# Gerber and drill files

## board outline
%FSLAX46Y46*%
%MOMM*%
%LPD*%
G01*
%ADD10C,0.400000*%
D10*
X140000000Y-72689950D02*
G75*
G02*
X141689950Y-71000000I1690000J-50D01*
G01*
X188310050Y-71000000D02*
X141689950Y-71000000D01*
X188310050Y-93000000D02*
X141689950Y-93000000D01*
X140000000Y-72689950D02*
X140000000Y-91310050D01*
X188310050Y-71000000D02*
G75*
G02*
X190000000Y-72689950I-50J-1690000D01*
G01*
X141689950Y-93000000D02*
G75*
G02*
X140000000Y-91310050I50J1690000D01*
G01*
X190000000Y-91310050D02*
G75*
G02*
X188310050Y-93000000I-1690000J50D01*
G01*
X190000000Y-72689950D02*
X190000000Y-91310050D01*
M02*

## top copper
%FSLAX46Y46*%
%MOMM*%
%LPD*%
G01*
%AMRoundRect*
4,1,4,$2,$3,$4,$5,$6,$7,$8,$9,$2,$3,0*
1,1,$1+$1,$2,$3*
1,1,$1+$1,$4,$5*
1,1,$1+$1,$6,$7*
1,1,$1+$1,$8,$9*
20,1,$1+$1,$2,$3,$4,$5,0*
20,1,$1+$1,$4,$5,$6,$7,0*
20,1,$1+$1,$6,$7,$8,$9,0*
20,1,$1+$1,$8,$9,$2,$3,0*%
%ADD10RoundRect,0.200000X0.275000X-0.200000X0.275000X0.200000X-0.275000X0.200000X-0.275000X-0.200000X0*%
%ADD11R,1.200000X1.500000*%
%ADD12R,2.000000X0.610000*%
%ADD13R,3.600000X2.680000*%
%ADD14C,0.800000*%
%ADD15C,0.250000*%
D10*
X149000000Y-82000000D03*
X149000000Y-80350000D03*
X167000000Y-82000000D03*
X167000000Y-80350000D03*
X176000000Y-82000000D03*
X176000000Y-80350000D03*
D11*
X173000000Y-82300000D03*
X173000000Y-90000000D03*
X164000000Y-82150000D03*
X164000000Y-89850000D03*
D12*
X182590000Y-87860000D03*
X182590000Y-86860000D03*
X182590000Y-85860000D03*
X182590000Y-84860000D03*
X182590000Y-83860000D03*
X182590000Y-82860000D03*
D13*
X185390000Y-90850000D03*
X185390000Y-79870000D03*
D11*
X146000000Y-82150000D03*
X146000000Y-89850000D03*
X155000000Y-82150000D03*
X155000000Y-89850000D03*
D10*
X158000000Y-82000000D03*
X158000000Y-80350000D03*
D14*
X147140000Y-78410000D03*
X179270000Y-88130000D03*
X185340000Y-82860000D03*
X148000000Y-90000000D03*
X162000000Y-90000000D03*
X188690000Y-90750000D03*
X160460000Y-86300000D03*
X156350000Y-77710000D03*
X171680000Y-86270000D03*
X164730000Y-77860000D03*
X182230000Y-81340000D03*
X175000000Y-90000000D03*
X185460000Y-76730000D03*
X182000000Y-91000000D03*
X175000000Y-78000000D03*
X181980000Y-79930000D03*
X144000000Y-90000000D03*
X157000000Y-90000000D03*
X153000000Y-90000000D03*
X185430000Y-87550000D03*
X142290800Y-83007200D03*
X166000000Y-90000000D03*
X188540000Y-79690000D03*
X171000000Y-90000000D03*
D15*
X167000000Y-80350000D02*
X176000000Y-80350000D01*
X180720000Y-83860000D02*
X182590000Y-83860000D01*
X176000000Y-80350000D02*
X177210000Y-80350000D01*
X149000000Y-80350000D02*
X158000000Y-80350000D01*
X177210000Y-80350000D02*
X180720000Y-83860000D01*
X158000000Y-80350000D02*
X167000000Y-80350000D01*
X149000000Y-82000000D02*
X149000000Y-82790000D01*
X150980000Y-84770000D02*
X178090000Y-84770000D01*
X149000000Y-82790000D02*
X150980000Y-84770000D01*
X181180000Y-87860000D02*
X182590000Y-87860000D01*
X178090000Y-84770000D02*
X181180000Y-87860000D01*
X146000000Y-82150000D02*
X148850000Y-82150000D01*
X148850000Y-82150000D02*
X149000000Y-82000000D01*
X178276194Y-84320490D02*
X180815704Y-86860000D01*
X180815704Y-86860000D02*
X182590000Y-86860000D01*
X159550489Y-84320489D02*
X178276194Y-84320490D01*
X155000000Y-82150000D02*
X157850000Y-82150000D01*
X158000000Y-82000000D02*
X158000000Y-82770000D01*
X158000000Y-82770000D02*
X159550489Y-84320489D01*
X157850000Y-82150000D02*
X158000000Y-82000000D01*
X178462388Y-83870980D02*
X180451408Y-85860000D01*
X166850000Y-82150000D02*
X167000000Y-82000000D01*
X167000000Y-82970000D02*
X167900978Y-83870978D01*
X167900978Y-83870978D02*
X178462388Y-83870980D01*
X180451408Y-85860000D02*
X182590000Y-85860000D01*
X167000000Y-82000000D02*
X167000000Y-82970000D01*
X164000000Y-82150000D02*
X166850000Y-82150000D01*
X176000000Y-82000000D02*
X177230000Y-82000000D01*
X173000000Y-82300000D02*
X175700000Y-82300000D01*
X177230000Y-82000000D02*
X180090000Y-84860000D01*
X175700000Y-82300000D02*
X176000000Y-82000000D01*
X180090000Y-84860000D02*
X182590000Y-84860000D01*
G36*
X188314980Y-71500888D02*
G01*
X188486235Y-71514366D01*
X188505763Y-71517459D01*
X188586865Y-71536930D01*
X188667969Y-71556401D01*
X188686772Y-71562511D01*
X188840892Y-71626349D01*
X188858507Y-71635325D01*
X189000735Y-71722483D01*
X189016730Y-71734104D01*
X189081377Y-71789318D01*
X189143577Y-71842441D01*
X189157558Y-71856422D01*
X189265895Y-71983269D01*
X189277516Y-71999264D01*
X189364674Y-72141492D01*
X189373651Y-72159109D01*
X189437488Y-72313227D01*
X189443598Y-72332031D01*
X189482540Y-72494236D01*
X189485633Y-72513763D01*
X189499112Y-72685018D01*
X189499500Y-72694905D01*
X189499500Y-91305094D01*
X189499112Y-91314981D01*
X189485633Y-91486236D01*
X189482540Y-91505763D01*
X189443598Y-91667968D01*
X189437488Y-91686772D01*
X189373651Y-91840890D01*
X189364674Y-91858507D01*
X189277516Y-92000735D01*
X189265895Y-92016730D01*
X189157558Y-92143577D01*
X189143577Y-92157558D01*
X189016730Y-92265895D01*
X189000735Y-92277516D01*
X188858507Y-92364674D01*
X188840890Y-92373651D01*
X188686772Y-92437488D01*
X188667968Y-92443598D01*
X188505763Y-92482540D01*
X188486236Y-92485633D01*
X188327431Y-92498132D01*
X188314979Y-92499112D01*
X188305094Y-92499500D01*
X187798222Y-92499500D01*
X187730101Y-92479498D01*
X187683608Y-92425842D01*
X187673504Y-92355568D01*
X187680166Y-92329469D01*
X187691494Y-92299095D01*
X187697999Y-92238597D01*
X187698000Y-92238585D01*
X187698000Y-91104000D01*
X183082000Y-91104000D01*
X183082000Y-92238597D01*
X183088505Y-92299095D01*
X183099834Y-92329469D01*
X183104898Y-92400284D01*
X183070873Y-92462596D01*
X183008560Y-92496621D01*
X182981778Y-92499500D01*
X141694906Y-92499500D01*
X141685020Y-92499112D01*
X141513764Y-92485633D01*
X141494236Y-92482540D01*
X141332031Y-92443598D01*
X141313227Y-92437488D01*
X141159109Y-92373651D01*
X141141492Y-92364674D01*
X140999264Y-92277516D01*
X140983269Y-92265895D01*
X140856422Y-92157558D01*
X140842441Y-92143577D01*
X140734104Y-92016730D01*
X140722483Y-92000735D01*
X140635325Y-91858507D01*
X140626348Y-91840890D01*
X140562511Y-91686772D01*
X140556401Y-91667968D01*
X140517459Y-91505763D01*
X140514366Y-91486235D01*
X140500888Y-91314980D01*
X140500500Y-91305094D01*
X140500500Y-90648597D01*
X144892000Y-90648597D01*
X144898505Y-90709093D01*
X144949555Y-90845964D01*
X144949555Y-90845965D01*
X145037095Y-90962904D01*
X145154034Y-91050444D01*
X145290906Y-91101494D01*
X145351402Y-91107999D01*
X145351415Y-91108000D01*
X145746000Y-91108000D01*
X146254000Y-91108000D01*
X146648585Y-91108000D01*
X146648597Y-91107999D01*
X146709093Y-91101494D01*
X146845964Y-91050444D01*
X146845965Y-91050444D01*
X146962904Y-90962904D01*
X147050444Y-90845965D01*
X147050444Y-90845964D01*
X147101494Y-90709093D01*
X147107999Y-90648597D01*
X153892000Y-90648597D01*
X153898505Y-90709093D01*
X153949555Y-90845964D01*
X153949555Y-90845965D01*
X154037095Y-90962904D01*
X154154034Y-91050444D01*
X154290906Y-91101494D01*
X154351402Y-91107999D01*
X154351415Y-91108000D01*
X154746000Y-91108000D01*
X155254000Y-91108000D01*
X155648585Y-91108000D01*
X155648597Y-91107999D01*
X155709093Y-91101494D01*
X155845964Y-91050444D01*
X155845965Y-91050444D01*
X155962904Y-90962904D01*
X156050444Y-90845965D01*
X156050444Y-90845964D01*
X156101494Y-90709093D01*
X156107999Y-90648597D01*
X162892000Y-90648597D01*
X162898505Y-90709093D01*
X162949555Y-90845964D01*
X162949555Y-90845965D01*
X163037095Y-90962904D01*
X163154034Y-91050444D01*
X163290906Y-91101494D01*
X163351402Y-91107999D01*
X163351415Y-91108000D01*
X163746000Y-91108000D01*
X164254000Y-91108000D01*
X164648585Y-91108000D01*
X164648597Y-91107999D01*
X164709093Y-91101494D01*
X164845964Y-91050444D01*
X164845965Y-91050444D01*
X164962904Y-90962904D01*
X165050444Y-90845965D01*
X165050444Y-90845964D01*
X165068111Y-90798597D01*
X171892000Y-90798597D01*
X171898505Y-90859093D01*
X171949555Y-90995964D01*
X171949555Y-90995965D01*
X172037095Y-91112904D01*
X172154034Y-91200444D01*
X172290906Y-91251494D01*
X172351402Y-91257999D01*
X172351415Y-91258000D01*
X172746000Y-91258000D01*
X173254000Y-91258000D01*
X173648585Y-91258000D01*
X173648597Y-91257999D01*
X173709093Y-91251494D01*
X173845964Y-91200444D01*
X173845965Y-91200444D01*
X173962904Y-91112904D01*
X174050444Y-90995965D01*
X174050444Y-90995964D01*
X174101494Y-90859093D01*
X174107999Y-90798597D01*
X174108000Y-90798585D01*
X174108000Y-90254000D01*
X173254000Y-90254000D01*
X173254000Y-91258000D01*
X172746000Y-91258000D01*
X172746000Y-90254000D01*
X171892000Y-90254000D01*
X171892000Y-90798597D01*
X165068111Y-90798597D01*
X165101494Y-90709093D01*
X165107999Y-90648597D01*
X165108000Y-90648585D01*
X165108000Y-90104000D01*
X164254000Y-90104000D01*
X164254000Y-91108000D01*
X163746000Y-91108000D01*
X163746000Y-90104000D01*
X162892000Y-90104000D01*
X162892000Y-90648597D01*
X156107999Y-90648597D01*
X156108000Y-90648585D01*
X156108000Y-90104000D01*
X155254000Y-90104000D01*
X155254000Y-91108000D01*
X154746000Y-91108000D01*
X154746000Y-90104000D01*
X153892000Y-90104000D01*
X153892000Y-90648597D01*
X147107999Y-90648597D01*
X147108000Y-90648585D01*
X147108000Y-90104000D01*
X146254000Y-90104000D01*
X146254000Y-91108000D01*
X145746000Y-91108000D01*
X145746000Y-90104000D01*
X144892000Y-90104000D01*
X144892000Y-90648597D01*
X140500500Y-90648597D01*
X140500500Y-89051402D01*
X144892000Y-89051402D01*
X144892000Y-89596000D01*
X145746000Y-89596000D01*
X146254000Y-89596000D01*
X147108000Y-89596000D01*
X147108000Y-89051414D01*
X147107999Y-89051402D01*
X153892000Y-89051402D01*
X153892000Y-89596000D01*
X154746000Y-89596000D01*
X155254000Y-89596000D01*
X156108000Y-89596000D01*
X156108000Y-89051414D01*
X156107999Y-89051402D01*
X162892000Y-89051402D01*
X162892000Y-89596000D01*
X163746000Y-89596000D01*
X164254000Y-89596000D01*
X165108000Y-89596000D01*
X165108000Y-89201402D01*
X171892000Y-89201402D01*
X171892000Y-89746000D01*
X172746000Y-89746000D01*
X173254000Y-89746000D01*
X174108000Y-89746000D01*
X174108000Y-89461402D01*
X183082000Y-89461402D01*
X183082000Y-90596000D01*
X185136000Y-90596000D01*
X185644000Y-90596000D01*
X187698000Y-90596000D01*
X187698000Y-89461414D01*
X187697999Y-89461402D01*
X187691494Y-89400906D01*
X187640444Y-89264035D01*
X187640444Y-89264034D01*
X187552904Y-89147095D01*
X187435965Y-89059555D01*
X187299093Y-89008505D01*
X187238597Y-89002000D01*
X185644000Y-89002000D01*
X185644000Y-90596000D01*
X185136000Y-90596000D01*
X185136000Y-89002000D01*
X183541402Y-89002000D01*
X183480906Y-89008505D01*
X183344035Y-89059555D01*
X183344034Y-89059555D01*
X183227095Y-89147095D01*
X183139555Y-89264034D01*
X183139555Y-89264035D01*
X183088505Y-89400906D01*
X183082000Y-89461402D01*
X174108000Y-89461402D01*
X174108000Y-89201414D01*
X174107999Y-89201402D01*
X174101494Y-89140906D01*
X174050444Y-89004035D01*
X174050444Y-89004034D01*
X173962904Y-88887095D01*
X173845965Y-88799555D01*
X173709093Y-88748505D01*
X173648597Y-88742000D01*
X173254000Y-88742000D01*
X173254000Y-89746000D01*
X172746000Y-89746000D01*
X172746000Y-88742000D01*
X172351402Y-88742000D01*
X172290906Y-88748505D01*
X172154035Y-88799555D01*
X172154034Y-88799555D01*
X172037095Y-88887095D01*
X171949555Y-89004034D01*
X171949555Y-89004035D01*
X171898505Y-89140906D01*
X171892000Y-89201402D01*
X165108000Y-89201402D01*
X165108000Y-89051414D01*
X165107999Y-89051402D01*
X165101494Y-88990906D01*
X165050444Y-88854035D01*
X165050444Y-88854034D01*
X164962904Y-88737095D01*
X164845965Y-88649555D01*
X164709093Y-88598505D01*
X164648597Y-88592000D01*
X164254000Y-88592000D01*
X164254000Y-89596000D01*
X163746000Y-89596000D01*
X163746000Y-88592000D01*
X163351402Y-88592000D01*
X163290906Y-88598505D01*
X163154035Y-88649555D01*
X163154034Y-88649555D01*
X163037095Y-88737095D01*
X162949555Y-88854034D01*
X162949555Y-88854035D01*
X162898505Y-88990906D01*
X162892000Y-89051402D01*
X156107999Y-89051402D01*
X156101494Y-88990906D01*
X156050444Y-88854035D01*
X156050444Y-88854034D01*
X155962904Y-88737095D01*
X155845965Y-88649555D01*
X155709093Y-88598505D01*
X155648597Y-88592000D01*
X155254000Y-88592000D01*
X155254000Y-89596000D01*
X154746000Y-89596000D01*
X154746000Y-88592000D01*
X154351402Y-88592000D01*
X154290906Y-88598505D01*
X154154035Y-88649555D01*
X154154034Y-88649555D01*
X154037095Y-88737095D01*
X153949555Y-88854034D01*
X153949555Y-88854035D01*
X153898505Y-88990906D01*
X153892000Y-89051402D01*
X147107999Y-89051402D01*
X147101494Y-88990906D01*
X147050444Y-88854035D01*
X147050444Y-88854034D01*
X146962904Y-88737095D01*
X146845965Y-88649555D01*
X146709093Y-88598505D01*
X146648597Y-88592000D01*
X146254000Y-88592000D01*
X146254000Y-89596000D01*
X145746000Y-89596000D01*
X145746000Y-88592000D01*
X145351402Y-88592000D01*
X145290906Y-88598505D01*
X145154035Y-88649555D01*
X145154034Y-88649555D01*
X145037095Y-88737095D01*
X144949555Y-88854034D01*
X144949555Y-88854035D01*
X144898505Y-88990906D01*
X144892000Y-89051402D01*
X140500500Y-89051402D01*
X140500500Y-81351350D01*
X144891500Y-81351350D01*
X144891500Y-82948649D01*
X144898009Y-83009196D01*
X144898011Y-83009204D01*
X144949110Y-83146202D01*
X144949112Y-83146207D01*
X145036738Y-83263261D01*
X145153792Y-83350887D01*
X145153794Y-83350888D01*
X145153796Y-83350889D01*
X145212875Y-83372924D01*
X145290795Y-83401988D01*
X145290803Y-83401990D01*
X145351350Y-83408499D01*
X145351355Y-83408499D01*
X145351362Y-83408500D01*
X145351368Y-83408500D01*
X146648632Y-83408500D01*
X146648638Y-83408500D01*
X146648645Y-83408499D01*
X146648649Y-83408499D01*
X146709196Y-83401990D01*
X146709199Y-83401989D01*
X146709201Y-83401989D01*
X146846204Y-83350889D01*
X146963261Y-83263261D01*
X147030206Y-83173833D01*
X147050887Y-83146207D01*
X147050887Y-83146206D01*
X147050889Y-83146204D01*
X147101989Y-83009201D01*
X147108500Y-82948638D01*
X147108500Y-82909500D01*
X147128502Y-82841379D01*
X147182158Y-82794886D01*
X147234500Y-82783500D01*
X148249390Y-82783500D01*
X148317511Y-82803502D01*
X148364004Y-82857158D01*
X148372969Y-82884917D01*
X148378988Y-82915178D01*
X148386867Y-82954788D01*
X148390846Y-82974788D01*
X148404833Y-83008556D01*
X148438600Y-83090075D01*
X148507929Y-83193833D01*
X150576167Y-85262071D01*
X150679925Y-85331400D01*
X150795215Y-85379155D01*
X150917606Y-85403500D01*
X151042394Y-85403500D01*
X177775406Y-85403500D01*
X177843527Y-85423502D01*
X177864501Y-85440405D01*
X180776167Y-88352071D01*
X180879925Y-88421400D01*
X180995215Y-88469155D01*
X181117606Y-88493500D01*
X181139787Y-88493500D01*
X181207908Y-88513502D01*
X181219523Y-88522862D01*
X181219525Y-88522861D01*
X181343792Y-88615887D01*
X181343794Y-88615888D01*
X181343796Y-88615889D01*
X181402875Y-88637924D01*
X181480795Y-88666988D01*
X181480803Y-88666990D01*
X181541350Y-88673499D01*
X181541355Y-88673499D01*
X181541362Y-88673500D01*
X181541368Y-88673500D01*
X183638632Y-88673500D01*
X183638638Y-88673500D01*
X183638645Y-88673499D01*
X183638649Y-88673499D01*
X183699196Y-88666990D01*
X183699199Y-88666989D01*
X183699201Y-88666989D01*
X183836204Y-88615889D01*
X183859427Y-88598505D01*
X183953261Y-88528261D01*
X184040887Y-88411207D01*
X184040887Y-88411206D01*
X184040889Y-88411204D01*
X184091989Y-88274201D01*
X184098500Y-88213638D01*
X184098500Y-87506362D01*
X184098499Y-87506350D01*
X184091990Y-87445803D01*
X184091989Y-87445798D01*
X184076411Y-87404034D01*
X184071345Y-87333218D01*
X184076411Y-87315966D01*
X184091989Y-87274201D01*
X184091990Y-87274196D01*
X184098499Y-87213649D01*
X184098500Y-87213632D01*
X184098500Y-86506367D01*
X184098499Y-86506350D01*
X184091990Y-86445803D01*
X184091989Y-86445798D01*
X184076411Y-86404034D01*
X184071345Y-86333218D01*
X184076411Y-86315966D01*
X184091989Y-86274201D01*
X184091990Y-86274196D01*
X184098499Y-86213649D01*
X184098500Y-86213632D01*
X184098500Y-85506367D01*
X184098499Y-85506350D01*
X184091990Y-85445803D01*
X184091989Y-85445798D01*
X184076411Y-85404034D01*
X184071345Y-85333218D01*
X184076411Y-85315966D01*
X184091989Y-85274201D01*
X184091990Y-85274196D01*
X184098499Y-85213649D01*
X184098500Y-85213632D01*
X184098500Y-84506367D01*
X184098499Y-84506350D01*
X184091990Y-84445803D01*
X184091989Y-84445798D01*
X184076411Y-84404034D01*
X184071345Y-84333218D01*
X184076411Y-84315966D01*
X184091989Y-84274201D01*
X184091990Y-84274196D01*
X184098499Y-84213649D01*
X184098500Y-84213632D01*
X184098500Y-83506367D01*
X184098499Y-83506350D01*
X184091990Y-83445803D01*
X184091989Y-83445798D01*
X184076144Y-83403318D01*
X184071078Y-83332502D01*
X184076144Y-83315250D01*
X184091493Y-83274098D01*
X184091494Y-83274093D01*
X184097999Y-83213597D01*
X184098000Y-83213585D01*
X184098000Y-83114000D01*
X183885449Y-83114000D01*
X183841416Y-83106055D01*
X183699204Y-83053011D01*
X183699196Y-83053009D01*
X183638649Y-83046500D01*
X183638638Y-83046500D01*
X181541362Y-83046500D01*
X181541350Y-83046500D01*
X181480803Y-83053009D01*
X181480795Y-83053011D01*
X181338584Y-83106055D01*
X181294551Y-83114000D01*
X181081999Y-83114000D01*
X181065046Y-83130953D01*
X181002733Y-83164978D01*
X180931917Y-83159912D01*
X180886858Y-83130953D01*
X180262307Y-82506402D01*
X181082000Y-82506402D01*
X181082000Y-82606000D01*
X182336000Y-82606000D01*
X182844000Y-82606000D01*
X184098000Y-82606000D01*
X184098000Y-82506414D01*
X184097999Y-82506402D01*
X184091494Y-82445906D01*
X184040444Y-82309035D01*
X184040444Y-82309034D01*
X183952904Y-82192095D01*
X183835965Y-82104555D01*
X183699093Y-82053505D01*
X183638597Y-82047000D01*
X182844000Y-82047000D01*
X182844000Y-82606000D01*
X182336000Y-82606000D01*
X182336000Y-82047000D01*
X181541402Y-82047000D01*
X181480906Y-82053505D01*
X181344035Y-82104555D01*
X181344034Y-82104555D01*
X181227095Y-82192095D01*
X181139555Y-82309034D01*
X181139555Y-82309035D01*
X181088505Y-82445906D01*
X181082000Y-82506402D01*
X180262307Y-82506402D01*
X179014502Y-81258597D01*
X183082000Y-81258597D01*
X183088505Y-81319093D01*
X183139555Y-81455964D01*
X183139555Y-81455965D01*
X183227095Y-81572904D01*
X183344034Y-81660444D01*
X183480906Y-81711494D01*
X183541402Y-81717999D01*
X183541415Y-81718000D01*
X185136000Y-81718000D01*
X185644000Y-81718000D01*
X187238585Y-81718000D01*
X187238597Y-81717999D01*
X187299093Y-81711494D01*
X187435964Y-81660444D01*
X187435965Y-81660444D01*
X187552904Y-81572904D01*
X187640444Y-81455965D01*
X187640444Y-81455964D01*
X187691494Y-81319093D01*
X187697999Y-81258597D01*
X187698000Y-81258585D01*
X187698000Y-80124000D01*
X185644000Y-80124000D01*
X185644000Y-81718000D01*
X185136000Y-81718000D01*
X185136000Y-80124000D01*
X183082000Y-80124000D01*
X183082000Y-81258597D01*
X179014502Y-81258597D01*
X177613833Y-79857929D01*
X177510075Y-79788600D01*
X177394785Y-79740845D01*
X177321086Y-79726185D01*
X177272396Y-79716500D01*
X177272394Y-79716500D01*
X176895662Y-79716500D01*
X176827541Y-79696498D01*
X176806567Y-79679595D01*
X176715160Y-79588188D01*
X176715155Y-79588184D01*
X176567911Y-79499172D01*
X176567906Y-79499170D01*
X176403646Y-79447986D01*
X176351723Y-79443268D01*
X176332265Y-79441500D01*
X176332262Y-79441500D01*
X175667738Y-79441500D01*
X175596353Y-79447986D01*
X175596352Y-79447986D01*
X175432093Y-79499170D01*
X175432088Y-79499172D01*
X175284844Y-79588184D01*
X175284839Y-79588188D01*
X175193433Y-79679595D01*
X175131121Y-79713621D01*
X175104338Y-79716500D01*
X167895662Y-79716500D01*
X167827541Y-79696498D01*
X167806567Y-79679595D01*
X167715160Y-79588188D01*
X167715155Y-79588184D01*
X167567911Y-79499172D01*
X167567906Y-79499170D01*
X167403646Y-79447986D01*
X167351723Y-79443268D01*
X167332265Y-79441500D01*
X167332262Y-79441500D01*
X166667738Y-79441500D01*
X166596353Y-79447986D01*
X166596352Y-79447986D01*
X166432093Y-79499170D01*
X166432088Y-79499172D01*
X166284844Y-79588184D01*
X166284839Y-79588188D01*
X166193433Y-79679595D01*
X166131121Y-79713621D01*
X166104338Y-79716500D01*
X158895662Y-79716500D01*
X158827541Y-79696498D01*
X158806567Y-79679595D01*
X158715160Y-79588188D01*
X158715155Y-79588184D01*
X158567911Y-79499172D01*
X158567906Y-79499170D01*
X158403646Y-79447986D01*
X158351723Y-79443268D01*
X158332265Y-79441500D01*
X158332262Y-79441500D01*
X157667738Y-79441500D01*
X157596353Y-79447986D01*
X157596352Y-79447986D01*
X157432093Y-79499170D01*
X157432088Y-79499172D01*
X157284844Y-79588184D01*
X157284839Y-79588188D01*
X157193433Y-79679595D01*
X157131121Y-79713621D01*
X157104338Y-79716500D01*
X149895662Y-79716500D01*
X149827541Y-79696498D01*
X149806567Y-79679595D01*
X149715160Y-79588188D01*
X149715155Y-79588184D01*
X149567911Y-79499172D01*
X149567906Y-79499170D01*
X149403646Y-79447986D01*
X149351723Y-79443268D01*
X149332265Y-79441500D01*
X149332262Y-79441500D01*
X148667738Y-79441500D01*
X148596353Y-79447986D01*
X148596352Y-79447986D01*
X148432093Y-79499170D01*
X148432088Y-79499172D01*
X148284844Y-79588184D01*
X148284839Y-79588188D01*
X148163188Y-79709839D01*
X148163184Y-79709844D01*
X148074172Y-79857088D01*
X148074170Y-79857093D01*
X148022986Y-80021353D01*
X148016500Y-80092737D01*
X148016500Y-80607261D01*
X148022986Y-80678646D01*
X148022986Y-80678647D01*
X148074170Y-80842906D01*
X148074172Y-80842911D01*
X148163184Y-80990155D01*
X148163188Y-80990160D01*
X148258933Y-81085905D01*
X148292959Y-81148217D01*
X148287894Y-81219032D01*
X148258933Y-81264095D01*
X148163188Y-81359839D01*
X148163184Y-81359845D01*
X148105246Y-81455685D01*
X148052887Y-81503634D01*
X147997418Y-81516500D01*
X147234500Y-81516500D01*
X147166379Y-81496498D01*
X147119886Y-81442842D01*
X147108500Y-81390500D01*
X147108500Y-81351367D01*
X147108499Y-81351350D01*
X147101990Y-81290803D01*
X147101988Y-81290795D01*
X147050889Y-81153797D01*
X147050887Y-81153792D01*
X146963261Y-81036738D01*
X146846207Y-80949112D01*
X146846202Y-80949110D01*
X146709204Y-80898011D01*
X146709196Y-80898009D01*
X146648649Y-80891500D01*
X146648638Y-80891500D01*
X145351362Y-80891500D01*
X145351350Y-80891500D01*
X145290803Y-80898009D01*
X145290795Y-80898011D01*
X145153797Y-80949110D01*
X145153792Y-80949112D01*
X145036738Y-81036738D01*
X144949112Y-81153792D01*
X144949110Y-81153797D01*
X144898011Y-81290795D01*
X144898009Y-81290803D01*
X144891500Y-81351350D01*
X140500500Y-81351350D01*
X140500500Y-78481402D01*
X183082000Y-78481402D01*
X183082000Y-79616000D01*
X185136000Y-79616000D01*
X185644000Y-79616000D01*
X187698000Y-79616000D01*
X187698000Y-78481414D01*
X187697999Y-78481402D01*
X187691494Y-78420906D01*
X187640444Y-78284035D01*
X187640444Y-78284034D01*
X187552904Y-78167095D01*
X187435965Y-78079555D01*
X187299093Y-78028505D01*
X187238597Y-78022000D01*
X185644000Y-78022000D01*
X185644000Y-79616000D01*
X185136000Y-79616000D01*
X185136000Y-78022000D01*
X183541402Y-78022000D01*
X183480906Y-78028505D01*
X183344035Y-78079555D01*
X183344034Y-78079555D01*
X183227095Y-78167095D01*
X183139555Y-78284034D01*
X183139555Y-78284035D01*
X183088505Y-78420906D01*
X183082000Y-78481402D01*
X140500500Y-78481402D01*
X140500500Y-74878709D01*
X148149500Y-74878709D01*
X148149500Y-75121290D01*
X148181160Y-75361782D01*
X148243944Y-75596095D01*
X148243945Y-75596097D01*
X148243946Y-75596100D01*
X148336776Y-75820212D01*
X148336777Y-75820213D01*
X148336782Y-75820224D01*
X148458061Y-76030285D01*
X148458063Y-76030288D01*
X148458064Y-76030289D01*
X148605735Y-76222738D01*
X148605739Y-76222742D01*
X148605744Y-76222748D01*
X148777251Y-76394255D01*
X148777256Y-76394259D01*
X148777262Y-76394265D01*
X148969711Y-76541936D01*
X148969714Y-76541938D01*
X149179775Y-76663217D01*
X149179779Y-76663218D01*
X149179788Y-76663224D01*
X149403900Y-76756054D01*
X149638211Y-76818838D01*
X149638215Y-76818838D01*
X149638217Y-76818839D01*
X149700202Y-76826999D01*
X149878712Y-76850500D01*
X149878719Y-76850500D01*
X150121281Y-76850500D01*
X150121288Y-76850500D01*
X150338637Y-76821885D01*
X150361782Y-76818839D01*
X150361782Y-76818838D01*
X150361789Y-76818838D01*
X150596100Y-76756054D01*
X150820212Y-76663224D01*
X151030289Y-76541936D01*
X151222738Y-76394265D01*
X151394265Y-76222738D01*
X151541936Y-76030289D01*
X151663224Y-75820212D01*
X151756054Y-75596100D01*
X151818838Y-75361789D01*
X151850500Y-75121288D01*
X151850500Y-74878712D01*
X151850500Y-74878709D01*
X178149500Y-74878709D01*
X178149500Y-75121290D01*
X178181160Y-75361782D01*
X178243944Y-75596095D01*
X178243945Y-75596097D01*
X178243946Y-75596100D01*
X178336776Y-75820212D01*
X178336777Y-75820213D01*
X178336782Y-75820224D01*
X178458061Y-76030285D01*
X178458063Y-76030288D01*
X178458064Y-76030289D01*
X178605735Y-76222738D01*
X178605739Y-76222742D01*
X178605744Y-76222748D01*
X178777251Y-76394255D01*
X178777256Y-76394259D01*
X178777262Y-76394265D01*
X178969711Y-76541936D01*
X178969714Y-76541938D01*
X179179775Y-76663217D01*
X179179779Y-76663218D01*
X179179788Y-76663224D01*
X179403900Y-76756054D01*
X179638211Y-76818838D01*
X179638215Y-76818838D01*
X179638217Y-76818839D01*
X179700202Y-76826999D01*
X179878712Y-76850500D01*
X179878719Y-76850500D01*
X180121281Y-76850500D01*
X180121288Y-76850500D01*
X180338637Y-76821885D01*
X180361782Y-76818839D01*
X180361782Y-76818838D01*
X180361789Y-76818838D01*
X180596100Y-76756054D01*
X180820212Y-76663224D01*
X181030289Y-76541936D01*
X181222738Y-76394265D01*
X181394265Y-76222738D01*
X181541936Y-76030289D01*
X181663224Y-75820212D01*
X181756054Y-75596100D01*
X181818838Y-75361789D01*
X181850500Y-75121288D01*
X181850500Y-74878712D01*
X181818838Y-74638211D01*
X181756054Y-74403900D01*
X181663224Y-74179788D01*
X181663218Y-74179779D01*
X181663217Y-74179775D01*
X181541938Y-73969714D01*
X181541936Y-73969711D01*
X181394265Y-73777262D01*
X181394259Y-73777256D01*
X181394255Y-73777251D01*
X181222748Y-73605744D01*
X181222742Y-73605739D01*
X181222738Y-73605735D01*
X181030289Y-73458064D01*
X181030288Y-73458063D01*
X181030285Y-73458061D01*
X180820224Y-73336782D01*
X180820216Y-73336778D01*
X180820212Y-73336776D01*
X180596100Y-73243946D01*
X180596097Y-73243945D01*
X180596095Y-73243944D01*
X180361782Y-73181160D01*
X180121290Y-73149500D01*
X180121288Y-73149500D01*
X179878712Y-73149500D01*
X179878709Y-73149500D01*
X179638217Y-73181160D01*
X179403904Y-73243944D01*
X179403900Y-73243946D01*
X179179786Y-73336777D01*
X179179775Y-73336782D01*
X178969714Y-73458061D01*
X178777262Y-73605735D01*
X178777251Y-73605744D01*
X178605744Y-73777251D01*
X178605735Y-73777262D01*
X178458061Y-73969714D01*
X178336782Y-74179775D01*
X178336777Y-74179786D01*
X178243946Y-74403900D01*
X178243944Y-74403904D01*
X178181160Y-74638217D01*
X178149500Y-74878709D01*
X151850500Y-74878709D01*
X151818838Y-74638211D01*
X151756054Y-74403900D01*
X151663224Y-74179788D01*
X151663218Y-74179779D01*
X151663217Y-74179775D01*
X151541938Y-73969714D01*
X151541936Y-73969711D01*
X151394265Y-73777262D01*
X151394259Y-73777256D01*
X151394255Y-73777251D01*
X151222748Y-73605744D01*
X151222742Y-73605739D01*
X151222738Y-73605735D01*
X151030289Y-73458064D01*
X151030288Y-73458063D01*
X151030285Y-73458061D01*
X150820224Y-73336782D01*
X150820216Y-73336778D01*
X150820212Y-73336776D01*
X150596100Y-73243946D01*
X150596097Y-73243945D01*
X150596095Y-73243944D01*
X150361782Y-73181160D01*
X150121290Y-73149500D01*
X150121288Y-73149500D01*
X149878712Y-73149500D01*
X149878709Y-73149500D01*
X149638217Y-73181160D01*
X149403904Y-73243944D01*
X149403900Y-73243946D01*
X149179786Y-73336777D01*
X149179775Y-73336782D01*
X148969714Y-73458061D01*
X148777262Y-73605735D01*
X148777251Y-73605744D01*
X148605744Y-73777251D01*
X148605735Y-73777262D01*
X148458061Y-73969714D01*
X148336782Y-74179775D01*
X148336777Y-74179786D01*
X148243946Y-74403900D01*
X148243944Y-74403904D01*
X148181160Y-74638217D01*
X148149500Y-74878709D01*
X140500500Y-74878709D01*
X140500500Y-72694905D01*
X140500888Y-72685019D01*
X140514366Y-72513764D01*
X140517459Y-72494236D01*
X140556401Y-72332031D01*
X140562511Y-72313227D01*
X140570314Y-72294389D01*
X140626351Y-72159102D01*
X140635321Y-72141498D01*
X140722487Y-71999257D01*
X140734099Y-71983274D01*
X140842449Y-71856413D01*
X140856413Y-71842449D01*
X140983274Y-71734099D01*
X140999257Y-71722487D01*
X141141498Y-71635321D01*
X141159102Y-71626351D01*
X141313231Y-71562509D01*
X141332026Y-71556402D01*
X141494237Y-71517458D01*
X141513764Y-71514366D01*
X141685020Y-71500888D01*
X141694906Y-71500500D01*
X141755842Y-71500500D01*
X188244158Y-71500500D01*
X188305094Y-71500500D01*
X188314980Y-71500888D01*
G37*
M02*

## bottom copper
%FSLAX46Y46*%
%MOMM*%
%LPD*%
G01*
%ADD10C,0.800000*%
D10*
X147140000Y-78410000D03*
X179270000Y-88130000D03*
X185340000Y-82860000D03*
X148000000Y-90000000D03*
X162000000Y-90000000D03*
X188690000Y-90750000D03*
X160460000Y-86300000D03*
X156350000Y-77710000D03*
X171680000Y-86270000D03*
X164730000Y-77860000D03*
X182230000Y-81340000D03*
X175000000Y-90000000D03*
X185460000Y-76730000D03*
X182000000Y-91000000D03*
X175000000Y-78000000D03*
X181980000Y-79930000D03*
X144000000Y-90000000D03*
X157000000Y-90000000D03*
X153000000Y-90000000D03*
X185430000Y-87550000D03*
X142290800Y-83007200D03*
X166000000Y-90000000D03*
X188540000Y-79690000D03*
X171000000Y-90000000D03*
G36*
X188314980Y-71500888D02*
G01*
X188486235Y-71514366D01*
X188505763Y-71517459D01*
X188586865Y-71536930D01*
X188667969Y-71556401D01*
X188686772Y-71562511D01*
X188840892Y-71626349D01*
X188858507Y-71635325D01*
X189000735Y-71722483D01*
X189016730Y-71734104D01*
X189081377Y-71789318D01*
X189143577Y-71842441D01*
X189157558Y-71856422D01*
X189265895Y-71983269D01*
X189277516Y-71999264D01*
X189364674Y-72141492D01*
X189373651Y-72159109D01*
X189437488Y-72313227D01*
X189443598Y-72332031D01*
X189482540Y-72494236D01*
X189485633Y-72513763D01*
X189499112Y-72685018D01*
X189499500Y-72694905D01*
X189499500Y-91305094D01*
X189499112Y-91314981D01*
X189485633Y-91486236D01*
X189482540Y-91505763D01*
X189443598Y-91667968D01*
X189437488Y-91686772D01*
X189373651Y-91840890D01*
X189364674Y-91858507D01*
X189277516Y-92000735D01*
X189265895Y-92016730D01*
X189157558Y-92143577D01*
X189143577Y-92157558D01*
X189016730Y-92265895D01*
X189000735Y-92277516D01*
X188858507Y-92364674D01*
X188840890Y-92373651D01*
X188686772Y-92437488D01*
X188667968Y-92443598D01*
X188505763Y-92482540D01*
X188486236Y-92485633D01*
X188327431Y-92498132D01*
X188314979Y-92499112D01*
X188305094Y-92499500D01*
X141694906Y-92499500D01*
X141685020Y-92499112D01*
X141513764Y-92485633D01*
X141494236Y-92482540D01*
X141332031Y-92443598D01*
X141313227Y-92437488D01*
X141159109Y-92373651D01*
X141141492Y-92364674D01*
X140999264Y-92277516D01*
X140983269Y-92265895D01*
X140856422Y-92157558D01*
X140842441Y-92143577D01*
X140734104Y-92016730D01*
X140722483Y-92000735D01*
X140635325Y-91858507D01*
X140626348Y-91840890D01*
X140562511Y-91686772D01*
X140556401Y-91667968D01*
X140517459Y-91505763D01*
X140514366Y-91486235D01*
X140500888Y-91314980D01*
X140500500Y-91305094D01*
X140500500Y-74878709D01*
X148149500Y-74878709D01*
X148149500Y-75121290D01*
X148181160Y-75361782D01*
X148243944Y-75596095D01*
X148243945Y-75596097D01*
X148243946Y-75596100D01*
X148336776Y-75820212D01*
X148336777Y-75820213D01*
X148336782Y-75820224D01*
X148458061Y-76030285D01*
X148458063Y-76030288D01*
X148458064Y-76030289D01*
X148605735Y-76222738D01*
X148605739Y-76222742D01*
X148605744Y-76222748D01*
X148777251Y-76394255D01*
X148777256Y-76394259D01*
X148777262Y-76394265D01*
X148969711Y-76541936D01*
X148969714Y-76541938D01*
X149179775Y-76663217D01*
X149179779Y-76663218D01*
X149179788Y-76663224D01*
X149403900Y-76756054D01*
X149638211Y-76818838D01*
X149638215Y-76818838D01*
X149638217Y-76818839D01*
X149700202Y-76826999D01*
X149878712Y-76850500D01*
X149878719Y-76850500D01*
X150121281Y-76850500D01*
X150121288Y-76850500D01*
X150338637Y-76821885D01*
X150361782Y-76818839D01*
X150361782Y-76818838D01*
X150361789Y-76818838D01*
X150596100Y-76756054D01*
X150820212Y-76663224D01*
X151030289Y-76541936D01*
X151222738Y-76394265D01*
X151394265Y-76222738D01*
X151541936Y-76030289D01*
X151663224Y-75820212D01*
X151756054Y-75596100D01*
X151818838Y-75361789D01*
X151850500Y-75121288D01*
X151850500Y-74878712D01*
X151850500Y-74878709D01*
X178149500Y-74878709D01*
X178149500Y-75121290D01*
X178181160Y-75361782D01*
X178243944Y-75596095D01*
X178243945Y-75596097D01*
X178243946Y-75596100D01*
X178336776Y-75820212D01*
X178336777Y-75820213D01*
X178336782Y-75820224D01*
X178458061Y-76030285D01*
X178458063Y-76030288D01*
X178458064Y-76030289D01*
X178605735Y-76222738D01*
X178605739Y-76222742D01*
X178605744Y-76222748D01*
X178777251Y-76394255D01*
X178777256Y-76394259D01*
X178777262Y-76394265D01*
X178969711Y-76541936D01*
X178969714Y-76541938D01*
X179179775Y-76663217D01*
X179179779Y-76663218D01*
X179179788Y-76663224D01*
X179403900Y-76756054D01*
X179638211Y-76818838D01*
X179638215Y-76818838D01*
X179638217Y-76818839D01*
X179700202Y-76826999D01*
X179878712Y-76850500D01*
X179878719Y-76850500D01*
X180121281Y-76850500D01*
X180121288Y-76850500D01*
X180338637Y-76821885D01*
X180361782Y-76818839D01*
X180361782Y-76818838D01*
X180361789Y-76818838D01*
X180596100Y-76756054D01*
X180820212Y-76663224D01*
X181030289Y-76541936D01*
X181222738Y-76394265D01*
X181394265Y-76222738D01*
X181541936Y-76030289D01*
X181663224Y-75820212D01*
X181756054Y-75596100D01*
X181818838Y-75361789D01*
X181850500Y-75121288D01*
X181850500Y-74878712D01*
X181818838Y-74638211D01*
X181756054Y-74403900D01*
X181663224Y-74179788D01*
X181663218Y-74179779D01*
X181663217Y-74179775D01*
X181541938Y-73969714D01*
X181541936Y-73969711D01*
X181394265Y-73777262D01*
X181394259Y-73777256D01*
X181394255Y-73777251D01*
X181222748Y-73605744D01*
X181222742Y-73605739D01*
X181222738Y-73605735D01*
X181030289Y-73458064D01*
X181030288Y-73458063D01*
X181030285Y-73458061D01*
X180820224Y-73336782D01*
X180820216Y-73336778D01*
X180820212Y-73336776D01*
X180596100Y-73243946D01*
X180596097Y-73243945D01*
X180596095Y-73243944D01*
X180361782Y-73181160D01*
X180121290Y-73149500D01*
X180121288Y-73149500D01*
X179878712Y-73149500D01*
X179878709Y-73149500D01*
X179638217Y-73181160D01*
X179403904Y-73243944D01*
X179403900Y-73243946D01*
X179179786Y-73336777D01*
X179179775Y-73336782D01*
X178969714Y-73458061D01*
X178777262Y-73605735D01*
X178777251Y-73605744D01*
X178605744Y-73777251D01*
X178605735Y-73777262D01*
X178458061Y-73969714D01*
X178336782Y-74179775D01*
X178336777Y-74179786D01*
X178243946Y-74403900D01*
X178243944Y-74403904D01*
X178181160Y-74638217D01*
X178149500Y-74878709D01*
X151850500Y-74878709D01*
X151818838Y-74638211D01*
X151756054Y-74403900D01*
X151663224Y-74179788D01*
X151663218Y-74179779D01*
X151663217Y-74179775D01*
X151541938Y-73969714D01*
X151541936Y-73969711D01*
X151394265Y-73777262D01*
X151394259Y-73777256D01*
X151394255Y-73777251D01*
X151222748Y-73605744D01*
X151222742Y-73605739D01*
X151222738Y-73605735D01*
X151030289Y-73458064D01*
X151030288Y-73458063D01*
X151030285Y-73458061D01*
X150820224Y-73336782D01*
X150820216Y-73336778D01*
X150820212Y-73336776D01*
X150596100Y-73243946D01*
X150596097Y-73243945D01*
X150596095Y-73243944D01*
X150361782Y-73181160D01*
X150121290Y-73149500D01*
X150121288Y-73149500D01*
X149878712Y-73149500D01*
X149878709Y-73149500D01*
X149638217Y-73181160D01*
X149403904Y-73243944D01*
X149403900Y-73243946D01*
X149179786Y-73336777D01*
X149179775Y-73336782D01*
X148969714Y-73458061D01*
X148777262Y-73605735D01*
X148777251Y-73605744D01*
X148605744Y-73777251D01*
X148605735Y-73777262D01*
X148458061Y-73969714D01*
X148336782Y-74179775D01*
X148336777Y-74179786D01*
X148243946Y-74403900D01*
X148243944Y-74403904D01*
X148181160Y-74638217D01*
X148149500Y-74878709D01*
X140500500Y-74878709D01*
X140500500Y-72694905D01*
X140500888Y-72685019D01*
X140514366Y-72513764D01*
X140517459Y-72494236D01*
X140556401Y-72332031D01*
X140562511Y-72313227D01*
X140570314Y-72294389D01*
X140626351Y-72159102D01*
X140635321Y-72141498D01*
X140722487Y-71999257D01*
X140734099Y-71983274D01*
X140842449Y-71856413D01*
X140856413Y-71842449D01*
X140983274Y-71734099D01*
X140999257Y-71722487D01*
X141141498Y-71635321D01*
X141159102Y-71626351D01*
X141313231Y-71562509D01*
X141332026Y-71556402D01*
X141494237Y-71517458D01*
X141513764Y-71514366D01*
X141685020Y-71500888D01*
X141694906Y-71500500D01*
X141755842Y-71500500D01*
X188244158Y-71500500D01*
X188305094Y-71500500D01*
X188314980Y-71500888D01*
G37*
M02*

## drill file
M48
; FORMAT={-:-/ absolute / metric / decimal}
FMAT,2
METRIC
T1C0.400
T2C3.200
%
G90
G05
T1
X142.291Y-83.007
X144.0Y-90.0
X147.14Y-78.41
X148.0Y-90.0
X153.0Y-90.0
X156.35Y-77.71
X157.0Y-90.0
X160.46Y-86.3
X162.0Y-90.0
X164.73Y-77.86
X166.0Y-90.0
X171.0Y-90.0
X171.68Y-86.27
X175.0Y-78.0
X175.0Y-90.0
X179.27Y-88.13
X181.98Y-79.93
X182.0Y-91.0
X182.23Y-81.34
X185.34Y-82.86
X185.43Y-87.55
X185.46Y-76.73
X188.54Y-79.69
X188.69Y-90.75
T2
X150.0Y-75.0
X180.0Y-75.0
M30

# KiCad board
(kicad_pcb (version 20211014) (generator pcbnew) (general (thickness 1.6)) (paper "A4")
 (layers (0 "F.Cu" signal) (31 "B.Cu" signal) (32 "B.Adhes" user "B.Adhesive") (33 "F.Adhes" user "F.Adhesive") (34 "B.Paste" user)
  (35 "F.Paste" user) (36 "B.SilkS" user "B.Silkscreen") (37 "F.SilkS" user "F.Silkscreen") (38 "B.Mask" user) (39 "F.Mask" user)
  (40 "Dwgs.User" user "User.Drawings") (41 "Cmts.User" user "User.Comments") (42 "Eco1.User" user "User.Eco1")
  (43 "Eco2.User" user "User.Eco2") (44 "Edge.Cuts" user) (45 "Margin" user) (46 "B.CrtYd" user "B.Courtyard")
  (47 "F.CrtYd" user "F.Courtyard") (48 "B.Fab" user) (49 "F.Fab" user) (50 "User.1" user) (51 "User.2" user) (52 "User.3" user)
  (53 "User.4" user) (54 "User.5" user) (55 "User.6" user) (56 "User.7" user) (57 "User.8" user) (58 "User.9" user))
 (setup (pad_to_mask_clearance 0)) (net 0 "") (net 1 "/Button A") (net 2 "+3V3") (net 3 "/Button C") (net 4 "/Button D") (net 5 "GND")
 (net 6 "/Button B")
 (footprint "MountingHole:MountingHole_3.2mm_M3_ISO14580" (layer "F.Cu") (at 150 75)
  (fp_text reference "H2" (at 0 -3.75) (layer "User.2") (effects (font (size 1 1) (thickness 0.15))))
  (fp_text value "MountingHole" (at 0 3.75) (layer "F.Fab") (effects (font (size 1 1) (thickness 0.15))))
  (pad "" np_thru_hole circle (at 0 0) (size 3.2 3.2) (drill 3.2) (layers *.Cu *.Mask)))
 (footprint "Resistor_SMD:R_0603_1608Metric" (layer "F.Cu") (at 149 81.175 90)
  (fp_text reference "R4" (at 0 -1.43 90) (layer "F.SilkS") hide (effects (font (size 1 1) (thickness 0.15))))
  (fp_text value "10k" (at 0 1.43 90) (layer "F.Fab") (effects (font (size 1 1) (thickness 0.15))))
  (pad "1" smd roundrect locked (at -0.825 0 90) (size 0.8 0.95) (layers "F.Cu" "F.Paste" "F.Mask") (roundrect_rratio 0.25)
   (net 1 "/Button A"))
  (pad "2" smd roundrect locked (at 0.825 0 90) (size 0.8 0.95) (layers "F.Cu" "F.Paste" "F.Mask") (roundrect_rratio 0.25) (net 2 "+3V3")))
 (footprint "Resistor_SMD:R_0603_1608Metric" (layer "F.Cu") (at 167 81.175 90)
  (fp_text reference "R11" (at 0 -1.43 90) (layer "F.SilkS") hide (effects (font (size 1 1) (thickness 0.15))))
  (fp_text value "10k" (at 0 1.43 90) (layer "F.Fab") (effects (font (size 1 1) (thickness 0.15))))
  (pad "1" smd roundrect locked (at -0.825 0 90) (size 0.8 0.95) (layers "F.Cu" "F.Paste" "F.Mask") (roundrect_rratio 0.25)
   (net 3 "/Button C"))
  (pad "2" smd roundrect locked (at 0.825 0 90) (size 0.8 0.95) (layers "F.Cu" "F.Paste" "F.Mask") (roundrect_rratio 0.25) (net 2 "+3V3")))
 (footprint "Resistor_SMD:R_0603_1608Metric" (layer "F.Cu") (at 176 81.175 90)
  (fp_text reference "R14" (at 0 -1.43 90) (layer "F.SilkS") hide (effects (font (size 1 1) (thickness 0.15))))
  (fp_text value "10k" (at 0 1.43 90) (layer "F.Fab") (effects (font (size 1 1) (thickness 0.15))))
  (pad "1" smd roundrect locked (at -0.825 0 90) (size 0.8 0.95) (layers "F.Cu" "F.Paste" "F.Mask") (roundrect_rratio 0.25)
   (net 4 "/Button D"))
  (pad "2" smd roundrect locked (at 0.825 0 90) (size 0.8 0.95) (layers "F.Cu" "F.Paste" "F.Mask") (roundrect_rratio 0.25) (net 2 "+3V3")))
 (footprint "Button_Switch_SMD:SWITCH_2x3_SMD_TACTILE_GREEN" (layer "F.Cu") (at 173 86.15 -90)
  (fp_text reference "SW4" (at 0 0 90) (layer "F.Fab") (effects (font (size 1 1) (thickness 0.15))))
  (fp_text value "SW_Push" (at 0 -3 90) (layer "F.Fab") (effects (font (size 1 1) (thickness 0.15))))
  (pad "1" smd rect (at -3.85 0 270) (size 1.5 1.2) (layers "F.Cu" "F.Paste" "F.Mask") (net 4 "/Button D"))
  (pad "2" smd rect (at 3.85 0 270) (size 1.5 1.2) (layers "F.Cu" "F.Paste" "F.Mask") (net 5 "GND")))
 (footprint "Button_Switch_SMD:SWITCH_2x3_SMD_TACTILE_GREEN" (layer "F.Cu") (at 164 86 -90)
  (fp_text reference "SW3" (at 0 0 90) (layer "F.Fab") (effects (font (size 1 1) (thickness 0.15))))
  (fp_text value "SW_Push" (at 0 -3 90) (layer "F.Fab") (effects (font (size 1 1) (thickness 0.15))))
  (pad "1" smd rect (at -3.85 0 270) (size 1.5 1.2) (layers "F.Cu" "F.Paste" "F.Mask") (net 3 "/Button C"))
  (pad "2" smd rect (at 3.85 0 270) (size 1.5 1.2) (layers "F.Cu" "F.Paste" "F.Mask") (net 5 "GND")))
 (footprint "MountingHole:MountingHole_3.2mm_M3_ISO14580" (layer "F.Cu") (at 180 75)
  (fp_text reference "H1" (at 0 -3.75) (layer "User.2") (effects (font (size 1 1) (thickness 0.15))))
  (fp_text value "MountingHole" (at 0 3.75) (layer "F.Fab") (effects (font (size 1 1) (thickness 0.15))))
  (pad "" np_thru_hole circle (at 0 0) (size 3.2 3.2) (drill 3.2) (layers *.Cu *.Mask)))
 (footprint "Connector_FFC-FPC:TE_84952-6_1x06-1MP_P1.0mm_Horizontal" (layer "F.Cu") (at 184.39 85.36 90)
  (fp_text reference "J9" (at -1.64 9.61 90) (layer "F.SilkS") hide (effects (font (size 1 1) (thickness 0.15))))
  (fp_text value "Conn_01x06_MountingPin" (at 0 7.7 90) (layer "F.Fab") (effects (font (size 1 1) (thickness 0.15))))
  (pad "1" smd rect locked (at -2.5 -1.8 90) (size 0.61 2) (layers "F.Cu" "F.Paste" "F.Mask") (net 1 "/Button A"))
  (pad "2" smd rect locked (at -1.5 -1.8 90) (size 0.61 2) (layers "F.Cu" "F.Paste" "F.Mask") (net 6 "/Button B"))
  (pad "3" smd rect locked (at -0.5 -1.8 90) (size 0.61 2) (layers "F.Cu" "F.Paste" "F.Mask") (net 3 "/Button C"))
  (pad "4" smd rect locked (at 0.5 -1.8 90) (size 0.61 2) (layers "F.Cu" "F.Paste" "F.Mask") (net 4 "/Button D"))
  (pad "5" smd rect locked (at 1.5 -1.8 90) (size 0.61 2) (layers "F.Cu" "F.Paste" "F.Mask") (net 2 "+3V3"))
  (pad "6" smd rect locked (at 2.5 -1.8 90) (size 0.61 2) (layers "F.Cu" "F.Paste" "F.Mask") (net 5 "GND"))
  (pad "MP" smd rect locked (at -5.49 1 90) (size 2.68 3.6) (layers "F.Cu" "F.Paste" "F.Mask") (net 5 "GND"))
  (pad "MP" smd rect locked (at 5.49 1 90) (size 2.68 3.6) (layers "F.Cu" "F.Paste" "F.Mask") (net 5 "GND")))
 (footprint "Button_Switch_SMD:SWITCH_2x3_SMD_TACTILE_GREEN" (layer "F.Cu") (at 146 86 -90)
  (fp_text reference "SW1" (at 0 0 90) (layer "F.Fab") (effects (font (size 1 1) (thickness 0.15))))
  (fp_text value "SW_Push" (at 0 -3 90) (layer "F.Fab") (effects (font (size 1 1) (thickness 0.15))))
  (pad "1" smd rect (at -3.85 0 270) (size 1.5 1.2) (layers "F.Cu" "F.Paste" "F.Mask") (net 1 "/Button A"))
  (pad "2" smd rect (at 3.85 0 270) (size 1.5 1.2) (layers "F.Cu" "F.Paste" "F.Mask") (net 5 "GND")))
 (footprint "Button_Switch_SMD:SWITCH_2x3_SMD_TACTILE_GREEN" (layer "F.Cu") (at 155 86 -90)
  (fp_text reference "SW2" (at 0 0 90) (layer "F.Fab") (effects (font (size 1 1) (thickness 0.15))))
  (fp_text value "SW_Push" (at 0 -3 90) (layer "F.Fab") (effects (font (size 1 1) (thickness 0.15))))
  (pad "1" smd rect (at -3.85 0 270) (size 1.5 1.2) (layers "F.Cu" "F.Paste" "F.Mask") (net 6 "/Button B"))
  (pad "2" smd rect (at 3.85 0 270) (size 1.5 1.2) (layers "F.Cu" "F.Paste" "F.Mask") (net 5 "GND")))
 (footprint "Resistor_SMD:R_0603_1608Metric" (layer "F.Cu") (at 158 81.175 90)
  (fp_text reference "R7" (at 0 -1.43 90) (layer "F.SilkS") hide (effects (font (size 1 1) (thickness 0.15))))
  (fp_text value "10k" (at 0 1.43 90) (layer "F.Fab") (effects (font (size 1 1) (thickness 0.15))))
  (pad "1" smd roundrect locked (at -0.825 0 90) (size 0.8 0.95) (layers "F.Cu" "F.Paste" "F.Mask") (roundrect_rratio 0.25)
   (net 6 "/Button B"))
  (pad "2" smd roundrect locked (at 0.825 0 90) (size 0.8 0.95) (layers "F.Cu" "F.Paste" "F.Mask") (roundrect_rratio 0.25) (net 2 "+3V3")))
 (gr_arc (start 140 72.68995) (mid 140.494975 71.494975) (end 141.68995 71) (layer "Edge.Cuts") (width 0.4))
 (gr_line (start 188.31005 71) (end 141.68995 71) (layer "Edge.Cuts") (width 0.4))
 (gr_line (start 188.31005 93) (end 141.68995 93) (layer "Edge.Cuts") (width 0.4))
 (gr_line (start 140 72.68995) (end 140 91.31005) (layer "Edge.Cuts") (width 0.4))
 (gr_arc (start 188.31005 71) (mid 189.505025 71.494975) (end 190 72.68995) (layer "Edge.Cuts") (width 0.4))
 (gr_arc (start 141.68995 93) (mid 140.494975 92.505025) (end 140 91.31005) (layer "Edge.Cuts") (width 0.4))
 (gr_arc (start 190 91.31005) (mid 189.505025 92.505025) (end 188.31005 93) (layer "Edge.Cuts") (width 0.4))
 (gr_line (start 190 72.68995) (end 190 91.31005) (layer "Edge.Cuts") (width 0.4))
 (via (at 147.14 78.41) (size 0.8) (drill 0.4) (layers "F.Cu" "B.Cu") (free) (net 5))
 (via (at 179.27 88.13) (size 0.8) (drill 0.4) (layers "F.Cu" "B.Cu") (free) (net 5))
 (via (at 185.34 82.86) (size 0.8) (drill 0.4) (layers "F.Cu" "B.Cu") (free) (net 5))
 (via (at 148 90) (size 0.8) (drill 0.4) (layers "F.Cu" "B.Cu") (free) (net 5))
 (via (at 162 90) (size 0.8) (drill 0.4) (layers "F.Cu" "B.Cu") (free) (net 5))
 (via (at 188.69 90.75) (size 0.8) (drill 0.4) (layers "F.Cu" "B.Cu") (free) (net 5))
 (via (at 160.46 86.3) (size 0.8) (drill 0.4) (layers "F.Cu" "B.Cu") (free) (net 5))
 (via (at 156.35 77.71) (size 0.8) (drill 0.4) (layers "F.Cu" "B.Cu") (free) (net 5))
 (via (at 171.68 86.27) (size 0.8) (drill 0.4) (layers "F.Cu" "B.Cu") (free) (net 5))
 (via (at 164.73 77.86) (size 0.8) (drill 0.4) (layers "F.Cu" "B.Cu") (free) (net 5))
 (via (at 182.23 81.34) (size 0.8) (drill 0.4) (layers "F.Cu" "B.Cu") (free) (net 5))
 (via (at 175 90) (size 0.8) (drill 0.4) (layers "F.Cu" "B.Cu") (free) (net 5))
 (via (at 185.46 76.73) (size 0.8) (drill 0.4) (layers "F.Cu" "B.Cu") (free) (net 5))
 (via (at 182 91) (size 0.8) (drill 0.4) (layers "F.Cu" "B.Cu") (free) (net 5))
 (via (at 175 78) (size 0.8) (drill 0.4) (layers "F.Cu" "B.Cu") (free) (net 5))
 (via (at 181.98 79.93) (size 0.8) (drill 0.4) (layers "F.Cu" "B.Cu") (free) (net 5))
 (via (at 144 90) (size 0.8) (drill 0.4) (layers "F.Cu" "B.Cu") (free) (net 5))
 (via (at 157 90) (size 0.8) (drill 0.4) (layers "F.Cu" "B.Cu") (free) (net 5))
 (via (at 153 90) (size 0.8) (drill 0.4) (layers "F.Cu" "B.Cu") (free) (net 5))
 (via (at 185.43 87.55) (size 0.8) (drill 0.4) (layers "F.Cu" "B.Cu") (free) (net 5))
 (via (at 142.2908 83.0072) (size 0.8) (drill 0.4) (layers "F.Cu" "B.Cu") (free) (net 5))
 (via (at 166 90) (size 0.8) (drill 0.4) (layers "F.Cu" "B.Cu") (free) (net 5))
 (via (at 188.54 79.69) (size 0.8) (drill 0.4) (layers "F.Cu" "B.Cu") (free) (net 5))
 (via (at 171 90) (size 0.8) (drill 0.4) (layers "F.Cu" "B.Cu") (free) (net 5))
 (segment (start 167 80.35) (end 176 80.35) (width 0.25) (layer "F.Cu") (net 2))
 (segment (start 180.72 83.86) (end 182.59 83.86) (width 0.25) (layer "F.Cu") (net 2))
 (segment (start 176 80.35) (end 177.21 80.35) (width 0.25) (layer "F.Cu") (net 2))
 (segment (start 149 80.35) (end 158 80.35) (width 0.25) (layer "F.Cu") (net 2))
 (segment (start 177.21 80.35) (end 180.72 83.86) (width 0.25) (layer "F.Cu") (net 2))
 (segment (start 158 80.35) (end 167 80.35) (width 0.25) (layer "F.Cu") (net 2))
 (segment (start 149 82) (end 149 82.79) (width 0.25) (layer "F.Cu") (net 1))
 (segment (start 150.98 84.77) (end 178.09 84.77) (width 0.25) (layer "F.Cu") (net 1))
 (segment (start 149 82.79) (end 150.98 84.77) (width 0.25) (layer "F.Cu") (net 1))
 (segment (start 181.18 87.86) (end 182.59 87.86) (width 0.25) (layer "F.Cu") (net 1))
 (segment (start 178.09 84.77) (end 181.18 87.86) (width 0.25) (layer "F.Cu") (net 1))
 (segment (start 146 82.15) (end 148.85 82.15) (width 0.25) (layer "F.Cu") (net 1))
 (segment (start 148.85 82.15) (end 149 82) (width 0.25) (layer "F.Cu") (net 1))
 (segment (start 178.276194 84.32049) (end 180.815704 86.86) (width 0.25) (layer "F.Cu") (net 6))
 (segment (start 180.815704 86.86) (end 182.59 86.86) (width 0.25) (layer "F.Cu") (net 6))
 (segment (start 159.550489 84.320489) (end 178.276194 84.32049) (width 0.25) (layer "F.Cu") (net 6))
 (segment (start 155 82.15) (end 157.85 82.15) (width 0.25) (layer "F.Cu") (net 6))
 (segment (start 158 82) (end 158 82.77) (width 0.25) (layer "F.Cu") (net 6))
 (segment (start 158 82.77) (end 159.550489 84.320489) (width 0.25) (layer "F.Cu") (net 6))
 (segment (start 157.85 82.15) (end 158 82) (width 0.25) (layer "F.Cu") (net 6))
 (segment (start 178.462388 83.87098) (end 180.451408 85.86) (width 0.25) (layer "F.Cu") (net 3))
 (segment (start 166.85 82.15) (end 167 82) (width 0.25) (layer "F.Cu") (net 3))
 (segment (start 167 82.97) (end 167.900978 83.870978) (width 0.25) (layer "F.Cu") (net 3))
 (segment (start 167.900978 83.870978) (end 178.462388 83.87098) (width 0.25) (layer "F.Cu") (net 3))
 (segment (start 180.451408 85.86) (end 182.59 85.86) (width 0.25) (layer "F.Cu") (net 3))
 (segment (start 167 82) (end 167 82.97) (width 0.25) (layer "F.Cu") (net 3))
 (segment (start 164 82.15) (end 166.85 82.15) (width 0.25) (layer "F.Cu") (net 3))
 (segment (start 176 82) (end 177.23 82) (width 0.25) (layer "F.Cu") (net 4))
 (segment (start 173 82.3) (end 175.7 82.3) (width 0.25) (layer "F.Cu") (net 4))
 (segment (start 177.23 82) (end 180.09 84.86) (width 0.25) (layer "F.Cu") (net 4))
 (segment (start 175.7 82.3) (end 176 82) (width 0.25) (layer "F.Cu") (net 4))
 (segment (start 180.09 84.86) (end 182.59 84.86) (width 0.25) (layer "F.Cu") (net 4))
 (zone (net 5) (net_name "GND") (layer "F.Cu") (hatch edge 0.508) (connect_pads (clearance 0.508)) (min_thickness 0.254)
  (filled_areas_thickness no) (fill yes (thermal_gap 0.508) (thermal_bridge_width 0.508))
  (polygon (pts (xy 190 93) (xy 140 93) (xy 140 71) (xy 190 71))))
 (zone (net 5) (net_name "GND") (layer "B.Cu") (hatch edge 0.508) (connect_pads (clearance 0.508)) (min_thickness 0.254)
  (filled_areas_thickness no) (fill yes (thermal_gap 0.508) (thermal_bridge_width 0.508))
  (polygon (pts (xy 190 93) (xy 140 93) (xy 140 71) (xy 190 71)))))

